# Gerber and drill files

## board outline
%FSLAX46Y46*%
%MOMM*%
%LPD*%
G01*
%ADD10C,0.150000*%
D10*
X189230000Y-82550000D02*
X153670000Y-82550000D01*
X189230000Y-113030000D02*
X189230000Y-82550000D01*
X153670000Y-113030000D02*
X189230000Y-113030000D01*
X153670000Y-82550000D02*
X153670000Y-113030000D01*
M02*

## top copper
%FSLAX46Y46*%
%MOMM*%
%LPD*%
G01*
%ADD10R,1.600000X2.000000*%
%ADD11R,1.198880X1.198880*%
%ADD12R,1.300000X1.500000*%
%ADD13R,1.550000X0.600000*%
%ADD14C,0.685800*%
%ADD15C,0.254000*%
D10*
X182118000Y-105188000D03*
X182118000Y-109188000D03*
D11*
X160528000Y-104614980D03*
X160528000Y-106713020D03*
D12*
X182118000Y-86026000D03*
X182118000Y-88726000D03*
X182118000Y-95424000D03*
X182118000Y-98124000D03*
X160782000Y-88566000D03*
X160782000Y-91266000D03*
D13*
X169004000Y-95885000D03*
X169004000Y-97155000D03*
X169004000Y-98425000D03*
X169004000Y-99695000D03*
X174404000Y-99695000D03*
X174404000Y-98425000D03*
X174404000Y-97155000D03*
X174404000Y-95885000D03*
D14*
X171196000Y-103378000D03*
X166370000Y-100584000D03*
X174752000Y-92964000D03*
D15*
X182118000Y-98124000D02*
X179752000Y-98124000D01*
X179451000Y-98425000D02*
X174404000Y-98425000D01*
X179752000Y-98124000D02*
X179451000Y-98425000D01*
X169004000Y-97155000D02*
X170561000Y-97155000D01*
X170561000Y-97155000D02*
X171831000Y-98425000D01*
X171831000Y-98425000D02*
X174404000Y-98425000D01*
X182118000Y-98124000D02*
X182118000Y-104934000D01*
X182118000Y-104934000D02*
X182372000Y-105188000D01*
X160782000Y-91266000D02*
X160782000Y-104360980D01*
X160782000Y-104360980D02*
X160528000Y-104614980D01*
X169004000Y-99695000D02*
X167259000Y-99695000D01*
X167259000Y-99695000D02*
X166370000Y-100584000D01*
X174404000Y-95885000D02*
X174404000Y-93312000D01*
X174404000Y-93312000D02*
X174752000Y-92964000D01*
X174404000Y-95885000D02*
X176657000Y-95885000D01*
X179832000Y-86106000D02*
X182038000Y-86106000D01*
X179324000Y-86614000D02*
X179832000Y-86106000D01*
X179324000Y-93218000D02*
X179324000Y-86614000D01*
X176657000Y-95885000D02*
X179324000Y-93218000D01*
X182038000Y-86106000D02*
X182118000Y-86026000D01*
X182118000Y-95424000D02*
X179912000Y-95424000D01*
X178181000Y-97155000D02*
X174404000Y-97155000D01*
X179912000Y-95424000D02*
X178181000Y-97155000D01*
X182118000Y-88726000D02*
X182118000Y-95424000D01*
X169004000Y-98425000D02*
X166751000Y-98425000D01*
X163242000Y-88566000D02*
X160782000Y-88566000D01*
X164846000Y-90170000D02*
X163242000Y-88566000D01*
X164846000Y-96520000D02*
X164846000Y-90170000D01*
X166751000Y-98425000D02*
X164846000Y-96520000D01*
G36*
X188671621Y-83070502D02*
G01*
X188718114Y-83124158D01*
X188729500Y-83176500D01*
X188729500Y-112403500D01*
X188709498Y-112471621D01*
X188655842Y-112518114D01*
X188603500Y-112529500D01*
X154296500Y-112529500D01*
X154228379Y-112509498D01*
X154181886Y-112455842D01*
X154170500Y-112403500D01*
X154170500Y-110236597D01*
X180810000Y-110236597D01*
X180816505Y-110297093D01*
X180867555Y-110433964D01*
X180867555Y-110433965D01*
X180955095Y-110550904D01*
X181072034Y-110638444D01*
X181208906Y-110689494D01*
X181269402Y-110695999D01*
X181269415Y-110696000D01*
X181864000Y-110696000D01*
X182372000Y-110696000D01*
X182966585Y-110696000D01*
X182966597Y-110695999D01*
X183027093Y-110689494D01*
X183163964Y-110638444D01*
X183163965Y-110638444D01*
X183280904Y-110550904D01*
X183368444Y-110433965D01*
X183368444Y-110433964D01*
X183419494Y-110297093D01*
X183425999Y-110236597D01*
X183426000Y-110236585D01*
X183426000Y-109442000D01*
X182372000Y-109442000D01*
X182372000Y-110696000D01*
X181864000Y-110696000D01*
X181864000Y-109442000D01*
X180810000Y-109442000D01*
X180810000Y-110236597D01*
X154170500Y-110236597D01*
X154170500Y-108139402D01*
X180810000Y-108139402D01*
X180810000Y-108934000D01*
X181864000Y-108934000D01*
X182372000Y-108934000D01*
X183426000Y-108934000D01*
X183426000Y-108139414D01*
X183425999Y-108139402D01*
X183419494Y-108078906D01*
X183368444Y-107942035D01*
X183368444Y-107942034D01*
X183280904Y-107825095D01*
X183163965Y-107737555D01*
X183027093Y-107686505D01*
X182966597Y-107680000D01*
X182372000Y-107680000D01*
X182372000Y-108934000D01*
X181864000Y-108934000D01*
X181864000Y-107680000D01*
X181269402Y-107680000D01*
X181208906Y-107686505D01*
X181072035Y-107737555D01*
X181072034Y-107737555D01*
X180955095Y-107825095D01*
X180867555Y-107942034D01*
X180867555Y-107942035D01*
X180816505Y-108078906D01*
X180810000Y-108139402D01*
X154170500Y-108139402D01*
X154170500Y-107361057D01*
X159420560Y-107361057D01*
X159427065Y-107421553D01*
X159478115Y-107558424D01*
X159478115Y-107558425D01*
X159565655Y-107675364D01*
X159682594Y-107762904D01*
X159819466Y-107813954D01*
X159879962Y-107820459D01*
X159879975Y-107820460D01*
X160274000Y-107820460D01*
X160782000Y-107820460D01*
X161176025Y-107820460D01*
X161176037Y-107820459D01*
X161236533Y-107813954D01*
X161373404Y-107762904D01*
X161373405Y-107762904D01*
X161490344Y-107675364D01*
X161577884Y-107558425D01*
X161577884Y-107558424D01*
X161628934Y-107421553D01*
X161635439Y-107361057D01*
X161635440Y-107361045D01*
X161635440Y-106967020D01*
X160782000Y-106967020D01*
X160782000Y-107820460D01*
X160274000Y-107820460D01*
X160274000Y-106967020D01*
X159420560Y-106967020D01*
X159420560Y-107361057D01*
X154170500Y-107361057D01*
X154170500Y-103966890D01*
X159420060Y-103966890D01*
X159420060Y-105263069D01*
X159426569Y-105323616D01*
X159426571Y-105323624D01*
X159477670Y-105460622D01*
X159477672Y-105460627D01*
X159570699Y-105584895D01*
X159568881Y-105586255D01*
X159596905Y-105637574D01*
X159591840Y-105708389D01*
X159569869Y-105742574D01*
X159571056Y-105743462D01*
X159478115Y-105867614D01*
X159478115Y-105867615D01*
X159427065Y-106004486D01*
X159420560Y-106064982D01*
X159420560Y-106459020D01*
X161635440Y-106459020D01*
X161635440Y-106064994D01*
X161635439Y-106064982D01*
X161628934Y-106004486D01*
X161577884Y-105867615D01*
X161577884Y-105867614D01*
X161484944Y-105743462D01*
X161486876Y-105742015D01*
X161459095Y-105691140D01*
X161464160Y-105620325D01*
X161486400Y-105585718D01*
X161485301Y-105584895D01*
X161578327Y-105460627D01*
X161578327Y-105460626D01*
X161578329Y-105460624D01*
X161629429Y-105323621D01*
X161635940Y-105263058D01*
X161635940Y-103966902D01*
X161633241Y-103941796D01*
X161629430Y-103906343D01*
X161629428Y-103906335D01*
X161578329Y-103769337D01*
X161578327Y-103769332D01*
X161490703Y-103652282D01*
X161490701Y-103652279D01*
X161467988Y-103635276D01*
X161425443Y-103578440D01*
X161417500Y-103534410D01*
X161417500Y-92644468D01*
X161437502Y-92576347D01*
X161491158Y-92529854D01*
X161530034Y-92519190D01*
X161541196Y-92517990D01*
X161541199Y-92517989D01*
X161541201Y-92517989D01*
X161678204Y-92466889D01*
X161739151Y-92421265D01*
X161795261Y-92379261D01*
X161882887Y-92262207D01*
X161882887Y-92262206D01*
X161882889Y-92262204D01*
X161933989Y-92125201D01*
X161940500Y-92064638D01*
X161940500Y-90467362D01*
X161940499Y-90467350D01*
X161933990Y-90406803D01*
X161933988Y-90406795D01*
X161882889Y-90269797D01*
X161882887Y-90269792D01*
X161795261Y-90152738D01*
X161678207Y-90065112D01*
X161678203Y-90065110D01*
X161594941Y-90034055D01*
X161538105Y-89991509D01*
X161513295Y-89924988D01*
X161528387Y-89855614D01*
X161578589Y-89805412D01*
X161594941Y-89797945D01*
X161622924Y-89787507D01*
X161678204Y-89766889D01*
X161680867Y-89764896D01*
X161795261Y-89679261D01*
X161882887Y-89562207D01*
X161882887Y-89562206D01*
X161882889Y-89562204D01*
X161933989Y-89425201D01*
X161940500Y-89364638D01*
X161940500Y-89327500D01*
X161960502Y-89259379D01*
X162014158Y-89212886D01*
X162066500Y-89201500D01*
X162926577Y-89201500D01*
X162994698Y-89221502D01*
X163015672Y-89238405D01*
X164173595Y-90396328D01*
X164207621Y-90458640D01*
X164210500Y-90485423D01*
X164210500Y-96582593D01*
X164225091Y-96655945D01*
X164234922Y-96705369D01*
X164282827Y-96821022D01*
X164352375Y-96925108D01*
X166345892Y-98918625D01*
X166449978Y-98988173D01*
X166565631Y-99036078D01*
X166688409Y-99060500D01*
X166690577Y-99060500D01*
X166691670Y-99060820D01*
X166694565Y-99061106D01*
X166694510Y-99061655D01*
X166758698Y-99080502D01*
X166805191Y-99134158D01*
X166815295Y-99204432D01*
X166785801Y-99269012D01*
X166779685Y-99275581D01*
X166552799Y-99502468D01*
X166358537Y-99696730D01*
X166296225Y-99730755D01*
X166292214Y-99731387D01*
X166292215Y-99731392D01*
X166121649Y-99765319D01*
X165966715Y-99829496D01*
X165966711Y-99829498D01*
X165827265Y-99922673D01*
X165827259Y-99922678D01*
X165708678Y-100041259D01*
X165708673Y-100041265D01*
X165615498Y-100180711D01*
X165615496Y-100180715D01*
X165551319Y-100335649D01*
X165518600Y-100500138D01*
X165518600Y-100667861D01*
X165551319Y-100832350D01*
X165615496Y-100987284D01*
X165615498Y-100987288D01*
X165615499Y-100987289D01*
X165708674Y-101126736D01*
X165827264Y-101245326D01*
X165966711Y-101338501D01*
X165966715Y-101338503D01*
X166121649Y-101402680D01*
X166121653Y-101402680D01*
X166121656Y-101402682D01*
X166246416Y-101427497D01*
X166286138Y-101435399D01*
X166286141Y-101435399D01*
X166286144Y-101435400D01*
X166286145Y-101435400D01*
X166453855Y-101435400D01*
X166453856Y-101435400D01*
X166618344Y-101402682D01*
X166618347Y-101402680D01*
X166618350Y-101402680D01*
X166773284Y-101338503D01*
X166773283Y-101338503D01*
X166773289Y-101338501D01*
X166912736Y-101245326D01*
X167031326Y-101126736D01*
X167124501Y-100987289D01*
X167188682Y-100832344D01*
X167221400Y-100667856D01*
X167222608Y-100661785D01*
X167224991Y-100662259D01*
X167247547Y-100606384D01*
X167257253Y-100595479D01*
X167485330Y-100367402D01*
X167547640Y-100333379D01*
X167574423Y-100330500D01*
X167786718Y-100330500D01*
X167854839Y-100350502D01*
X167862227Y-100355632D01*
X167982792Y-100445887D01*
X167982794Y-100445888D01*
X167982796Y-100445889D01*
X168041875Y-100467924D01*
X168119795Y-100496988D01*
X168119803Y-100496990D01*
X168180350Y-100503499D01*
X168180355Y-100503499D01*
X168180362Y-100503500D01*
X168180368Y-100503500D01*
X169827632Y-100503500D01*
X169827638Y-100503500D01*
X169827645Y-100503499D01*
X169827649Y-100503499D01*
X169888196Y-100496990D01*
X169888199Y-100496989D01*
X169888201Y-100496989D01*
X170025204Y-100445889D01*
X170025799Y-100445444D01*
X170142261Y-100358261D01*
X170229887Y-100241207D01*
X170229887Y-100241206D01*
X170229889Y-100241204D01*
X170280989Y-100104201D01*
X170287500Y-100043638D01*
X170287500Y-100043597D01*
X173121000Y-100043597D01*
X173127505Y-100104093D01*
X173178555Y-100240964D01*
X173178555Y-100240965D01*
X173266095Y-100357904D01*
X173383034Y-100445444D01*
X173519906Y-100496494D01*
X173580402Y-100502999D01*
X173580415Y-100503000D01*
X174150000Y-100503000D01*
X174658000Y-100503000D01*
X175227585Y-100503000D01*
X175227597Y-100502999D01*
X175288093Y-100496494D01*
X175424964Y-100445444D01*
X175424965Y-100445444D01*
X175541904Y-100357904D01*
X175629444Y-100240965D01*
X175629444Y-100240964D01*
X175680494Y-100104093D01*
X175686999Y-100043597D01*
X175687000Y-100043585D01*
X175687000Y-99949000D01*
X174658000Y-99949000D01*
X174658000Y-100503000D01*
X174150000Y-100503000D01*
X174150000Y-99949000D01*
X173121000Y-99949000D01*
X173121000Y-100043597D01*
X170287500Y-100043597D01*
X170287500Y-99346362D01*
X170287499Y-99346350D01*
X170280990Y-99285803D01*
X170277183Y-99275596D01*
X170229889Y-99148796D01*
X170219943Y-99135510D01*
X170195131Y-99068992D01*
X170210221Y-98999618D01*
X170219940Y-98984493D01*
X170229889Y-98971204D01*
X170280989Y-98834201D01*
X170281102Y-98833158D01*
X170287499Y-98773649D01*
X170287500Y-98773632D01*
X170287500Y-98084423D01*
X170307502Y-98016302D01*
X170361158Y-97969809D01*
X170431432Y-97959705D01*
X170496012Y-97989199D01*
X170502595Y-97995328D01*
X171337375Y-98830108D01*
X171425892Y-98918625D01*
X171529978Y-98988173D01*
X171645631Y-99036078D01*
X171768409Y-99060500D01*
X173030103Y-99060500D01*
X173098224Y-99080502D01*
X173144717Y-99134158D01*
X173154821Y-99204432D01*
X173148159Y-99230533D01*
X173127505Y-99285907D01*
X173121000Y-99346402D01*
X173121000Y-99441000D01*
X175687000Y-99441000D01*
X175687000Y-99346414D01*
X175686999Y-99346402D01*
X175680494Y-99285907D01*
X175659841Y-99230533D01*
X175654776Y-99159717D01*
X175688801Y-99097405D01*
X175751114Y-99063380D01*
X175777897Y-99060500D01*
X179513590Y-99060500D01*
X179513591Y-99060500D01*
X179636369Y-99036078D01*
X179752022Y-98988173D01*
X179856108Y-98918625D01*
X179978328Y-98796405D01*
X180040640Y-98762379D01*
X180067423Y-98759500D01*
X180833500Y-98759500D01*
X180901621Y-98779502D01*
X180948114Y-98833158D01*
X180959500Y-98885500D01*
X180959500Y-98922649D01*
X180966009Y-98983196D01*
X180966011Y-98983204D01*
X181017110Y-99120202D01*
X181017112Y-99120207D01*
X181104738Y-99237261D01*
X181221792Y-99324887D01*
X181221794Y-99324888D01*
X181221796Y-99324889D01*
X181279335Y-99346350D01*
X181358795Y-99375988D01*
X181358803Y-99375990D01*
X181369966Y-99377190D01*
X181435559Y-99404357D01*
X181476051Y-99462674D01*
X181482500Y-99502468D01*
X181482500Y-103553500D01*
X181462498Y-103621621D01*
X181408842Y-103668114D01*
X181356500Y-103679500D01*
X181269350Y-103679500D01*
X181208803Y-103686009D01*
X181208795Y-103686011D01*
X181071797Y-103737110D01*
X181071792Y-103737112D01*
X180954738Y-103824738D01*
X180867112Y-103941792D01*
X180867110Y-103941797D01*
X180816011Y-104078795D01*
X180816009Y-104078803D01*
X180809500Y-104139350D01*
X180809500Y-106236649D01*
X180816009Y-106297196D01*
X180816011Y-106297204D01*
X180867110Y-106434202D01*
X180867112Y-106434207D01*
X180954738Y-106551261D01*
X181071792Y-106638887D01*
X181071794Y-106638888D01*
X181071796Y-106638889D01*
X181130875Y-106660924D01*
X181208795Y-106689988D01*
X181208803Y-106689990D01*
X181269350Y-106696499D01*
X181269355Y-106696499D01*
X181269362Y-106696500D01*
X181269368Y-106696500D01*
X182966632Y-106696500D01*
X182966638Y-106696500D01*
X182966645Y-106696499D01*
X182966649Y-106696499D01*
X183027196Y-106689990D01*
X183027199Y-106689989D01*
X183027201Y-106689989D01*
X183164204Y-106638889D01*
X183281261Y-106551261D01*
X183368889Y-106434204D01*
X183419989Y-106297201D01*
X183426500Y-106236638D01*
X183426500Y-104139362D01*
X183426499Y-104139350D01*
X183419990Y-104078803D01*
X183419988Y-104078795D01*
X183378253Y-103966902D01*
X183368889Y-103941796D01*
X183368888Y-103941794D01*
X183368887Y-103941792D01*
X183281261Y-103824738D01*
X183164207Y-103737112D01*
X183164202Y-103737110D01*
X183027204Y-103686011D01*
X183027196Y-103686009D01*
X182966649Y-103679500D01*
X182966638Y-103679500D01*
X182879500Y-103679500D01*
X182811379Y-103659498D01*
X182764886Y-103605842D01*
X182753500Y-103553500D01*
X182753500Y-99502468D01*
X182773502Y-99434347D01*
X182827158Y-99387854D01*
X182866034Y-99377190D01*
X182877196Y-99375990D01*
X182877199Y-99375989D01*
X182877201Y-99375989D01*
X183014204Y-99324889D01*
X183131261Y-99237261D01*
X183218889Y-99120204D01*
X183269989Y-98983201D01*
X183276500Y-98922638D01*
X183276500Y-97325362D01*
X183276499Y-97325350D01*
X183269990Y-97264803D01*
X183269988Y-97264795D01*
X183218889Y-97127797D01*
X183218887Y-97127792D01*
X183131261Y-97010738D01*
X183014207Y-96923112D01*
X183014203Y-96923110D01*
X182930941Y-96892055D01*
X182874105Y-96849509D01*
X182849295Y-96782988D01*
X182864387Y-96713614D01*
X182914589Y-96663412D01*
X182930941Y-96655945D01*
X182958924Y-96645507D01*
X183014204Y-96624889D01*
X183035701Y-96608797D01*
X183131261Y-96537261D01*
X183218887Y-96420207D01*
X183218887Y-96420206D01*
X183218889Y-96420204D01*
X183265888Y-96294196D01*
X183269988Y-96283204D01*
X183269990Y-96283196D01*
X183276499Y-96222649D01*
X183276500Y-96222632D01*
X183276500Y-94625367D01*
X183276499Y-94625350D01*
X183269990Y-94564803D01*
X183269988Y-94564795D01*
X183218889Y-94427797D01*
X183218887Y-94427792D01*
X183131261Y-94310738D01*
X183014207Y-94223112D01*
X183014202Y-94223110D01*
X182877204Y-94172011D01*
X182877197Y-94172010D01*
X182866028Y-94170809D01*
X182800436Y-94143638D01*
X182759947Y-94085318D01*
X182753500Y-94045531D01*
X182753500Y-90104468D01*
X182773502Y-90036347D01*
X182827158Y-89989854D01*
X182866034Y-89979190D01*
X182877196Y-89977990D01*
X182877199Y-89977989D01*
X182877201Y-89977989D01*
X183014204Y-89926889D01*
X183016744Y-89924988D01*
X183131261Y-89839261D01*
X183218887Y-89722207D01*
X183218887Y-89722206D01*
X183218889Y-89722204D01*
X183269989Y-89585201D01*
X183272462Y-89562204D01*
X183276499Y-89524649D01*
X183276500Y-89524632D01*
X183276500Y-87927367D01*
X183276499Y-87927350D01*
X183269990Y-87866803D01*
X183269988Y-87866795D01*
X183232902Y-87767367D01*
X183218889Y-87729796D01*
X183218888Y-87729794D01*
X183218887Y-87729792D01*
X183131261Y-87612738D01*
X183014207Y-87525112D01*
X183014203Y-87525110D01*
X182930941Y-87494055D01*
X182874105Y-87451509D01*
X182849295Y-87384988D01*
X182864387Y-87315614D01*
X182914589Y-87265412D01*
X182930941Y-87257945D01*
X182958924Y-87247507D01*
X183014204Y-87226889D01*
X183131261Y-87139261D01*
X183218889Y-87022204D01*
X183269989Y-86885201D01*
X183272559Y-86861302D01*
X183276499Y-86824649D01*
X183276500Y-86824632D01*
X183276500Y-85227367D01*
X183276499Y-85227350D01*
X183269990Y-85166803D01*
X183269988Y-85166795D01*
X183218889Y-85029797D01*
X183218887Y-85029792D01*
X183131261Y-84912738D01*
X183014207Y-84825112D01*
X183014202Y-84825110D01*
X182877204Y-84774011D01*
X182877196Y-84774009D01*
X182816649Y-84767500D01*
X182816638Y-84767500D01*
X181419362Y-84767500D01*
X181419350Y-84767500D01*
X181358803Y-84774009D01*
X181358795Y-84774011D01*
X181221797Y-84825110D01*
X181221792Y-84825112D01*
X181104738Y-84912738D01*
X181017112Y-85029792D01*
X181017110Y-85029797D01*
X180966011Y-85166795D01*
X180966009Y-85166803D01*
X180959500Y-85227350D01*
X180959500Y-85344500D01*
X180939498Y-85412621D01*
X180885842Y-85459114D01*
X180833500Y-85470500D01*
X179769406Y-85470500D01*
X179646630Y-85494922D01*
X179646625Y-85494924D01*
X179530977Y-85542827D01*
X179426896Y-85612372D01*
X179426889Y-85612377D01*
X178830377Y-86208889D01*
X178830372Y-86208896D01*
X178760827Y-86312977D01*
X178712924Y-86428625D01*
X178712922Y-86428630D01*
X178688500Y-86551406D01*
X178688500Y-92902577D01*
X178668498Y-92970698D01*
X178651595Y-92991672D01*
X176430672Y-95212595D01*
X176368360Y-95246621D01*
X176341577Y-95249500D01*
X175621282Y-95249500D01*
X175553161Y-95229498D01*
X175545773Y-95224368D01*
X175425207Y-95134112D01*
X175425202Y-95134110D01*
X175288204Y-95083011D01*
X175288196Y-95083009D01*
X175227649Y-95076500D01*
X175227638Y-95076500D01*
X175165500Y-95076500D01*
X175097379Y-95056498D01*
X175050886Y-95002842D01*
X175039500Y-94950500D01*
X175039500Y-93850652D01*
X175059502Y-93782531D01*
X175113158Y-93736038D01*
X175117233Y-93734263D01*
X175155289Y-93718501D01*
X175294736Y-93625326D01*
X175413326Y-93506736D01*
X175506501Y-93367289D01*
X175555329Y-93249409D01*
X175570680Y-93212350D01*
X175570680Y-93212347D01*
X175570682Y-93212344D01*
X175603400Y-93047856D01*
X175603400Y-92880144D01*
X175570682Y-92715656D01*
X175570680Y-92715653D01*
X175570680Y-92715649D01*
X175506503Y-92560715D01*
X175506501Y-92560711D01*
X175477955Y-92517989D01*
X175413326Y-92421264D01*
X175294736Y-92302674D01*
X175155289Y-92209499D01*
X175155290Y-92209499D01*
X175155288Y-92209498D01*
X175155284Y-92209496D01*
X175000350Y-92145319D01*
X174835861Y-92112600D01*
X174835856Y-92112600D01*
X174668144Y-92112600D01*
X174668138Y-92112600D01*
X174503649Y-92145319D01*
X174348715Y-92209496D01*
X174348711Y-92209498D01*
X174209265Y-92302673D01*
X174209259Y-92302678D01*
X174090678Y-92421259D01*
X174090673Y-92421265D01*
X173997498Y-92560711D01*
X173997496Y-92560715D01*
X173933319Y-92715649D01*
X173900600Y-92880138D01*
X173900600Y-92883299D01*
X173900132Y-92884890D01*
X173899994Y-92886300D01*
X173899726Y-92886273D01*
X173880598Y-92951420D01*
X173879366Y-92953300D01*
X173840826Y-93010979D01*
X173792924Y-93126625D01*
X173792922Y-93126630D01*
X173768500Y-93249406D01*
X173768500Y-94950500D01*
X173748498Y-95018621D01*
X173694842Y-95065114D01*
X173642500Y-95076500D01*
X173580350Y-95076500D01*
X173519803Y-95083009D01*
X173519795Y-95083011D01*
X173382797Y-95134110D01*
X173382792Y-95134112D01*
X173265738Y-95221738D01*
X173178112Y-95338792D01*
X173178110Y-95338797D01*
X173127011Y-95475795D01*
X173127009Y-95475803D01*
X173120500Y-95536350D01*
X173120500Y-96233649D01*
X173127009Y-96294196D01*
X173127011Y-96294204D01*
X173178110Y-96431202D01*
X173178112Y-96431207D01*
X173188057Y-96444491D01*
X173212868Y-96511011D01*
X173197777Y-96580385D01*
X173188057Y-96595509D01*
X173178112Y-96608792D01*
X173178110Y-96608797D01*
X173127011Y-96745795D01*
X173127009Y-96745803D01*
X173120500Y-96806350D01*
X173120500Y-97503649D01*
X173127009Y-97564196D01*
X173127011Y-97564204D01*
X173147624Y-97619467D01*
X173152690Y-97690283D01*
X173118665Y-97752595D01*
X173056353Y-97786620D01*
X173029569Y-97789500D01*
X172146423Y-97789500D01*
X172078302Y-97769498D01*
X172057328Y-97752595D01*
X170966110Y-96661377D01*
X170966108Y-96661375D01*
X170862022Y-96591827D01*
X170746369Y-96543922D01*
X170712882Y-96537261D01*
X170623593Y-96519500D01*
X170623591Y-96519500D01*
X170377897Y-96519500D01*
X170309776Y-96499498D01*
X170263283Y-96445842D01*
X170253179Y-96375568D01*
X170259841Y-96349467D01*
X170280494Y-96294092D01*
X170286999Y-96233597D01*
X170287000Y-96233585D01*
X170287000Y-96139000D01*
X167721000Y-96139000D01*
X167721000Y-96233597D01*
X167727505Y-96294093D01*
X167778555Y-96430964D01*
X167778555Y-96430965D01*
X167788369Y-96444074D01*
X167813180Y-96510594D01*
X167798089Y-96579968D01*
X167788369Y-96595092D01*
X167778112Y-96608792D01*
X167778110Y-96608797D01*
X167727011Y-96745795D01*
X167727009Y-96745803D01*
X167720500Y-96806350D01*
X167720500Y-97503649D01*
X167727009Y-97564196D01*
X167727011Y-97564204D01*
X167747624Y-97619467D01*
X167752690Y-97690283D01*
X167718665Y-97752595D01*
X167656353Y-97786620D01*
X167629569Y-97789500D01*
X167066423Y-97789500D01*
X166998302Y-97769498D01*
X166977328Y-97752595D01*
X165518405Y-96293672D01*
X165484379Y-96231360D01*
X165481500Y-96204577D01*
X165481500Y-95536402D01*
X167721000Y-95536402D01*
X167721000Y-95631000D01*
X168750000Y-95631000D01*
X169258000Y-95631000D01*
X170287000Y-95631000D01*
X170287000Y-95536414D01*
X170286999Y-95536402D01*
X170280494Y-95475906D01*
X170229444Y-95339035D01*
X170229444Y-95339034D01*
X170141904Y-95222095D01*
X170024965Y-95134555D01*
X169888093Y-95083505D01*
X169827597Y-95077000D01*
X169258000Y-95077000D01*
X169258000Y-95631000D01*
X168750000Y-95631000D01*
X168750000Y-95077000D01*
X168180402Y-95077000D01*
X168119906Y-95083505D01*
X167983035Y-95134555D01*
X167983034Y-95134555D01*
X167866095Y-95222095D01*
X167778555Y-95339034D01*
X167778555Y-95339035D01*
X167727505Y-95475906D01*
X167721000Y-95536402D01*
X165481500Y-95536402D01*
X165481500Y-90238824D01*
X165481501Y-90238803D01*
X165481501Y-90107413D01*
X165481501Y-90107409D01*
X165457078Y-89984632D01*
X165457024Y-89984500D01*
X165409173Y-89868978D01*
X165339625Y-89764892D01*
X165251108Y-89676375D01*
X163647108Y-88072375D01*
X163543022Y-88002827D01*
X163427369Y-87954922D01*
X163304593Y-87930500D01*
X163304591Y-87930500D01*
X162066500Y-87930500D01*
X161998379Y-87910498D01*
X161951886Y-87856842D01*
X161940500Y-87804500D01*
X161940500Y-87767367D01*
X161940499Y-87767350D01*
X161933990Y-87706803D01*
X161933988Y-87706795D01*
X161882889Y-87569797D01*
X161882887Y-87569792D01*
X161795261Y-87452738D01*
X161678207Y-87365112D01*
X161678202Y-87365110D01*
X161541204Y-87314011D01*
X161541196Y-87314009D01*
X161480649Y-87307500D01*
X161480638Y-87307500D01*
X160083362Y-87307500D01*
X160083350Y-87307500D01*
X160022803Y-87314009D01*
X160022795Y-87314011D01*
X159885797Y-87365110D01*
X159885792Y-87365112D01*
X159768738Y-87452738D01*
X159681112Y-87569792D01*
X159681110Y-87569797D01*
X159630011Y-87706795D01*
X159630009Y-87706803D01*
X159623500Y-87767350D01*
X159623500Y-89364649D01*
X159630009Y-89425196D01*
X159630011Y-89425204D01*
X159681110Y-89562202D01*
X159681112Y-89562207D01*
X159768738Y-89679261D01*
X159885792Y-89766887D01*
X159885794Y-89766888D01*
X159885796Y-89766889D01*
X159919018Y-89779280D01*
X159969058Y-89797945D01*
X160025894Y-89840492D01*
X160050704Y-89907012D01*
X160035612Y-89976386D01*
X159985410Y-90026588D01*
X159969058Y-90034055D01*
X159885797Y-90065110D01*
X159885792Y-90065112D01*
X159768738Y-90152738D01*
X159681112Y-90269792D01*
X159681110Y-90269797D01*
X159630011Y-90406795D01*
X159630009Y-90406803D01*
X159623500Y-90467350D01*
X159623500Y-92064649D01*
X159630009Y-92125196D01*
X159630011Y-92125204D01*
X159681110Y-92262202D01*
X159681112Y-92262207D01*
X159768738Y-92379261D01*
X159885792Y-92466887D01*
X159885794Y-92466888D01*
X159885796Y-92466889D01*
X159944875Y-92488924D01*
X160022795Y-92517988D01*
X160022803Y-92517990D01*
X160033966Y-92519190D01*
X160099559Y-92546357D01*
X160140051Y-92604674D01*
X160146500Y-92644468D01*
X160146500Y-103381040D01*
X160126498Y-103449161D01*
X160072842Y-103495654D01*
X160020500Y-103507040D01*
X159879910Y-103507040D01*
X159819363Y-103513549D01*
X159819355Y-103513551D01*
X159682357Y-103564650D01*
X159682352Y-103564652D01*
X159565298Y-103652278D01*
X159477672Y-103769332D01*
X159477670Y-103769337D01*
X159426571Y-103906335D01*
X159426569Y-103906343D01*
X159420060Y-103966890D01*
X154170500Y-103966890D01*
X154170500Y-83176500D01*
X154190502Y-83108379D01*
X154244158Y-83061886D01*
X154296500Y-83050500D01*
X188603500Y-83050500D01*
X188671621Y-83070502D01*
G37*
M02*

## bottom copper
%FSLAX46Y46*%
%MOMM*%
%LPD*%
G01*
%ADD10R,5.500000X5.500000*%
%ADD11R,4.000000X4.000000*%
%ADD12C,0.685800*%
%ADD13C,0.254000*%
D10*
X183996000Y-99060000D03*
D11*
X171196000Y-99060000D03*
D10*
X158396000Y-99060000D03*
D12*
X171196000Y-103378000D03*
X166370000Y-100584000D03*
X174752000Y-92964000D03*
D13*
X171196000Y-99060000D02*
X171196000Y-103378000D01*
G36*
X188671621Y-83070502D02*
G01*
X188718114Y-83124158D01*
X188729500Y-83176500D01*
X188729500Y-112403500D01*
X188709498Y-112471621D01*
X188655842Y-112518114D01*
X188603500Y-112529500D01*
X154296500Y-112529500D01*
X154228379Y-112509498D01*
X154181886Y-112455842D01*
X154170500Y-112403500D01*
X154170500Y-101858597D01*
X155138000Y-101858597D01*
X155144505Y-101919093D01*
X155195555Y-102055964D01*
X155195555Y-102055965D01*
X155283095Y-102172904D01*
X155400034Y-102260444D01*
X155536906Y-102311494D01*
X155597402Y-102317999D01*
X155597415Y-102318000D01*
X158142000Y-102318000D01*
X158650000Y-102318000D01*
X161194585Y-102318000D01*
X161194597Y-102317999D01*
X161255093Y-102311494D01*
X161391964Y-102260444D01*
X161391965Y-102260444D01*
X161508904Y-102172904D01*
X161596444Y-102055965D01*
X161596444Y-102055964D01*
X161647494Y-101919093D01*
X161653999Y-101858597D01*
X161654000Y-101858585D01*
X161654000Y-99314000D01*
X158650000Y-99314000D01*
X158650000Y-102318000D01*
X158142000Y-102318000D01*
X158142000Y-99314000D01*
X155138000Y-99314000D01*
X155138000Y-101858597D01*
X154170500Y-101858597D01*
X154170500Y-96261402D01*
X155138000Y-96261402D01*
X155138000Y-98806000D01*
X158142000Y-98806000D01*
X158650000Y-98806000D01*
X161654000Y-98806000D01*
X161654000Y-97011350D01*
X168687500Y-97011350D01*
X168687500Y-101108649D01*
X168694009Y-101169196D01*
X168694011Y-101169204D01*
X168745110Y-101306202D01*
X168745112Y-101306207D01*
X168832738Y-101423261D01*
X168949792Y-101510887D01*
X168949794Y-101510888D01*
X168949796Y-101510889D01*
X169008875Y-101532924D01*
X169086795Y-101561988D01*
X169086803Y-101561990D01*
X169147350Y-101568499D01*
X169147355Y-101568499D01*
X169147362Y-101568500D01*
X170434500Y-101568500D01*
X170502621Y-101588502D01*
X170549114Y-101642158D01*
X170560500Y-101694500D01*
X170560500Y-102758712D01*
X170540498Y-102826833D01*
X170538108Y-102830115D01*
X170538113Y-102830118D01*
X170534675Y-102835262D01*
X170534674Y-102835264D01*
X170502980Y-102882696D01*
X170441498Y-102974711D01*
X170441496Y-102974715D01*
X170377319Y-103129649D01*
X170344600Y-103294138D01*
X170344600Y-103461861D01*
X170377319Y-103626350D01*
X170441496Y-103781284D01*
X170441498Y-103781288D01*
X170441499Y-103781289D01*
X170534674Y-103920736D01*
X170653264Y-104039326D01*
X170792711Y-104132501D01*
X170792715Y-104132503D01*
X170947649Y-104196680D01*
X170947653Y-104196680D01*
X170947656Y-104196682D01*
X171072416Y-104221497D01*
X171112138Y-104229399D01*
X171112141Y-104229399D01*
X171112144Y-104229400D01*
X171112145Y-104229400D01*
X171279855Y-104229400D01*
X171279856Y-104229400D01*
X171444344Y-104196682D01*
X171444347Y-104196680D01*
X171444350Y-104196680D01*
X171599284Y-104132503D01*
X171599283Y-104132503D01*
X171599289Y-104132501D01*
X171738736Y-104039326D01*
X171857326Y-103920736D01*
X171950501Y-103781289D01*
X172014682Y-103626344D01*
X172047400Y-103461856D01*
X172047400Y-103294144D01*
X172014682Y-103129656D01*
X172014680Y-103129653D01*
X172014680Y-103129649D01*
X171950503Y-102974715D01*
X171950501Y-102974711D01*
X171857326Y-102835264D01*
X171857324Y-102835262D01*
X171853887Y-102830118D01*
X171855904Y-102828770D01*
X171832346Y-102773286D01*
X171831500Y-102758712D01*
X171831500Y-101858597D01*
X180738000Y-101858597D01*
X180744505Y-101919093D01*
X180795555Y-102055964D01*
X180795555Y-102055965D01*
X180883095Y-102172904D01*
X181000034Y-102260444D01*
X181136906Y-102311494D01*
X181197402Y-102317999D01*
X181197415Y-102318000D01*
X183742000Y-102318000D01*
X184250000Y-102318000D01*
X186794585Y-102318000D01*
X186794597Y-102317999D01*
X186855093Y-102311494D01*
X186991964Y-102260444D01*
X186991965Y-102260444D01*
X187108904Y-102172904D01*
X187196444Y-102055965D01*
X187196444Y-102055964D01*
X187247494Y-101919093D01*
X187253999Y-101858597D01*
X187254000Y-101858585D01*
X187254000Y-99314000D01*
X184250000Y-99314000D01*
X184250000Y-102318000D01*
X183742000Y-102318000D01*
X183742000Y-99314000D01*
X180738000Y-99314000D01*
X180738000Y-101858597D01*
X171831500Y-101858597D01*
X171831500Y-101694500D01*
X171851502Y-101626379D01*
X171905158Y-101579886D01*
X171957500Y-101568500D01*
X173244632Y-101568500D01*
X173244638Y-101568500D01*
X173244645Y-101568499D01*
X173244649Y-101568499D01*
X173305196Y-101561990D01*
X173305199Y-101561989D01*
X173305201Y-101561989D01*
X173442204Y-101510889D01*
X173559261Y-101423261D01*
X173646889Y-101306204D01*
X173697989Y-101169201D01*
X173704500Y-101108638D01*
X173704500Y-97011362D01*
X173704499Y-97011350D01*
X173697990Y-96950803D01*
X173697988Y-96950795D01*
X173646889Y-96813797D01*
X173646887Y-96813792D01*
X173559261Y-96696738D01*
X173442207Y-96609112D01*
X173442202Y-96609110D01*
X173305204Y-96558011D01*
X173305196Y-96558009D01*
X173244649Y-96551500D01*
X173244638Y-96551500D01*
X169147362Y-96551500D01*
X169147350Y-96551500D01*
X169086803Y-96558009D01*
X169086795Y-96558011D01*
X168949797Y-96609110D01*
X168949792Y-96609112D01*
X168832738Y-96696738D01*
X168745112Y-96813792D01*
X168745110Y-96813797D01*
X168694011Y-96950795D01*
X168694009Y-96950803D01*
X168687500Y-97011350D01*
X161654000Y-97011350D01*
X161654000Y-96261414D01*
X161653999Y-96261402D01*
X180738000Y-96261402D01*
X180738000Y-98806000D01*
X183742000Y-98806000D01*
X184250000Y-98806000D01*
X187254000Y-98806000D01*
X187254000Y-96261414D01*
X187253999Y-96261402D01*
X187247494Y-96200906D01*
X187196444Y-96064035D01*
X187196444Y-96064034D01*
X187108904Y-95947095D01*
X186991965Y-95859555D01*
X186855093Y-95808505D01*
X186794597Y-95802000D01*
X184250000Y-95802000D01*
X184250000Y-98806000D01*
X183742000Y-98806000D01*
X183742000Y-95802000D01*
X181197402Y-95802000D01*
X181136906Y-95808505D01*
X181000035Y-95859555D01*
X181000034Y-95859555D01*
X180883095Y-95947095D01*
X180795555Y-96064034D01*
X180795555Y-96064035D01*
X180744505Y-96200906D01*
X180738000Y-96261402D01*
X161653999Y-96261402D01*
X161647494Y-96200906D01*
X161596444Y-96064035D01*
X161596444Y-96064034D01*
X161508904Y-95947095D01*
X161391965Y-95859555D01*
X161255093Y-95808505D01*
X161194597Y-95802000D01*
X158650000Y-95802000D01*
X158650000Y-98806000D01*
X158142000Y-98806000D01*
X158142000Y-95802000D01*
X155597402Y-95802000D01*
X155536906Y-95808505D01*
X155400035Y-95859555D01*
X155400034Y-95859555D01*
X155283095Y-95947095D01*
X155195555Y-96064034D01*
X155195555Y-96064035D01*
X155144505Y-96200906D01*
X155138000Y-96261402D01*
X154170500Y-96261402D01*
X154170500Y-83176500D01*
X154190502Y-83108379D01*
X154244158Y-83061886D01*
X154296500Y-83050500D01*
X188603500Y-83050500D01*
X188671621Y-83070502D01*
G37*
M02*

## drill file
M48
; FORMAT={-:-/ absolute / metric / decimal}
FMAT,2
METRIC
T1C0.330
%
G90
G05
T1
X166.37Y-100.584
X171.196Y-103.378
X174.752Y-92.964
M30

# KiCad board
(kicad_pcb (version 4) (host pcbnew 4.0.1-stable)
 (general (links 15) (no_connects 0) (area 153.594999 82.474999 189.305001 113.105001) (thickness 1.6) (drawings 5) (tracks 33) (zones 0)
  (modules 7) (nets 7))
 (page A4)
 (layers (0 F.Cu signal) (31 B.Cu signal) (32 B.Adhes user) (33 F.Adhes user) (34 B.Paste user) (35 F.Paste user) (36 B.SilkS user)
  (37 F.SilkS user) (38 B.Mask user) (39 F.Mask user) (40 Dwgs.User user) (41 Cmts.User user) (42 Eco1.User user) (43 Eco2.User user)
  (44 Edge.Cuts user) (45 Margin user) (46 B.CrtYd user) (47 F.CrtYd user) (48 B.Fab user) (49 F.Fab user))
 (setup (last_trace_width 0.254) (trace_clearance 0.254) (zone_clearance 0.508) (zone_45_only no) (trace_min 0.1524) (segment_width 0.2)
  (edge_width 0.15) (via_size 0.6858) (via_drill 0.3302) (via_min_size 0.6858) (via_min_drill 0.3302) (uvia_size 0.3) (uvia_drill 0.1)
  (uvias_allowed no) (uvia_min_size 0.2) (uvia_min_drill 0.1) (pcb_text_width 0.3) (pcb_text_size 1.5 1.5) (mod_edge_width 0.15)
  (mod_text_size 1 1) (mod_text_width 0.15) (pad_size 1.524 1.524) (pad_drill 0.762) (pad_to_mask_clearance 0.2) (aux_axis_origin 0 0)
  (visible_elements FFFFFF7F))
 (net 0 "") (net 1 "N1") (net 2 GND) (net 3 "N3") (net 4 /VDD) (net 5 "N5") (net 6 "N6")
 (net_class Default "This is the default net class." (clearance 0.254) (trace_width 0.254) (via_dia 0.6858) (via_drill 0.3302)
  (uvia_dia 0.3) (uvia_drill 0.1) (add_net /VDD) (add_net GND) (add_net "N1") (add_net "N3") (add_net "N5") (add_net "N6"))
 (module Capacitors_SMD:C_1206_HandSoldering (layer F.Cu) (at 182.118 107.188 270)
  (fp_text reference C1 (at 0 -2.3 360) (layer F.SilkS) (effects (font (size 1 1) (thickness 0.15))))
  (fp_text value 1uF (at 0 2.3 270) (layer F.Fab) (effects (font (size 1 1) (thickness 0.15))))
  (pad 1 smd rect (at -2 0 270) (size 2 1.6) (layers F.Cu F.Paste F.Mask) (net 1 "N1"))
  (pad 2 smd rect (at 2 0 270) (size 2 1.6) (layers F.Cu F.Paste F.Mask) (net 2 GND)))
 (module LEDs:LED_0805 (layer F.Cu) (at 160.528 105.664 90)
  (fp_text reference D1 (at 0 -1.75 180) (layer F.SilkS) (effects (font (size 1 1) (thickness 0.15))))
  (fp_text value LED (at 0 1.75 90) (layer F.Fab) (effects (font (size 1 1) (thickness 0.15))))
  (pad 2 smd rect (at 1.04902 0 270) (size 1.19888 1.19888) (layers F.Cu F.Paste F.Mask) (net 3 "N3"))
  (pad 1 smd rect (at -1.04902 0 270) (size 1.19888 1.19888) (layers F.Cu F.Paste F.Mask) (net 2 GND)))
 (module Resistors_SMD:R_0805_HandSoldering (layer F.Cu) (at 182.118 87.376 270)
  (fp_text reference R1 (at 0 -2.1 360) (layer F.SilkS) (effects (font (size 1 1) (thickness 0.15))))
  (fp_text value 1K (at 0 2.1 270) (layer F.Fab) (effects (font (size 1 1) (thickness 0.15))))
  (pad 1 smd rect (at -1.35 0 270) (size 1.5 1.3) (layers F.Cu F.Paste F.Mask) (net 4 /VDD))
  (pad 2 smd rect (at 1.35 0 270) (size 1.5 1.3) (layers F.Cu F.Paste F.Mask) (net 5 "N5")))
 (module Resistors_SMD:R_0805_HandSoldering (layer F.Cu) (at 182.118 96.774 270)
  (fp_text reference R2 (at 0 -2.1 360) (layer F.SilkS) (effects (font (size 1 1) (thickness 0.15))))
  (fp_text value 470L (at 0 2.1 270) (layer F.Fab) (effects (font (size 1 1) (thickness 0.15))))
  (pad 1 smd rect (at -1.35 0 270) (size 1.5 1.3) (layers F.Cu F.Paste F.Mask) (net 5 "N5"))
  (pad 2 smd rect (at 1.35 0 270) (size 1.5 1.3) (layers F.Cu F.Paste F.Mask) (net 1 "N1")))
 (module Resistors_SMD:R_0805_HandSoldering (layer F.Cu) (at 160.782 89.916 270)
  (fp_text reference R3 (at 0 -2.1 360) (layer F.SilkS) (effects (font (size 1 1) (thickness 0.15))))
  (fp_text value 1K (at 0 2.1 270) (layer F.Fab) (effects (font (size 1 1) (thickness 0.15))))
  (pad 1 smd rect (at -1.35 0 270) (size 1.5 1.3) (layers F.Cu F.Paste F.Mask) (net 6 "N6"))
  (pad 2 smd rect (at 1.35 0 270) (size 1.5 1.3) (layers F.Cu F.Paste F.Mask) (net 3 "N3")))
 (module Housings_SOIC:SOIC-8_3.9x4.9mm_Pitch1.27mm (layer F.Cu) (at 171.704 97.79)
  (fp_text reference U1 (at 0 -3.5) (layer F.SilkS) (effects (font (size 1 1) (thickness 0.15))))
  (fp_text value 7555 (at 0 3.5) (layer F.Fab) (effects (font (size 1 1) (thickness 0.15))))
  (pad 1 smd rect (at -2.7 -1.905) (size 1.55 0.6) (layers F.Cu F.Paste F.Mask) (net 2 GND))
  (pad 2 smd rect (at -2.7 -0.635) (size 1.55 0.6) (layers F.Cu F.Paste F.Mask) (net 1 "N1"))
  (pad 3 smd rect (at -2.7 0.635) (size 1.55 0.6) (layers F.Cu F.Paste F.Mask) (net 6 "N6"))
  (pad 4 smd rect (at -2.7 1.905) (size 1.55 0.6) (layers F.Cu F.Paste F.Mask) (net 4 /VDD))
  (pad 5 smd rect (at 2.7 1.905) (size 1.55 0.6) (layers F.Cu F.Paste F.Mask) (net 2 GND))
  (pad 6 smd rect (at 2.7 0.635) (size 1.55 0.6) (layers F.Cu F.Paste F.Mask) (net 1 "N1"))
  (pad 7 smd rect (at 2.7 -0.635) (size 1.55 0.6) (layers F.Cu F.Paste F.Mask) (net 5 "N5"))
  (pad 8 smd rect (at 2.7 -1.905) (size 1.55 0.6) (layers F.Cu F.Paste F.Mask) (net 4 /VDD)))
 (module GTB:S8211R (layer B.Cu) (at 171.196 99.06)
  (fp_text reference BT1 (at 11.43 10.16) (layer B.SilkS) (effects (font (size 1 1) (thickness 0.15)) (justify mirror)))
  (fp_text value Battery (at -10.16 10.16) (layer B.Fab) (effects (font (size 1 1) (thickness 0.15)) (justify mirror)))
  (pad 1 smd rect (at 12.8 0) (size 5.5 5.5) (layers B.Cu B.Paste B.Mask) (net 4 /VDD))
  (pad 2 smd rect (at 0 0) (size 4 4) (layers B.Cu B.Paste B.Mask) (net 2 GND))
  (pad 1 smd rect (at -12.8 0) (size 5.5 5.5) (layers B.Cu B.Paste B.Mask) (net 4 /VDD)))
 (gr_line (start 189.23 82.55) (end 153.67 82.55) (angle 90) (layer Edge.Cuts) (width 0.15))
 (gr_line (start 189.23 113.03) (end 189.23 82.55) (angle 90) (layer Edge.Cuts) (width 0.15))
 (gr_line (start 153.67 113.03) (end 189.23 113.03) (angle 90) (layer Edge.Cuts) (width 0.15))
 (gr_line (start 153.67 82.55) (end 153.67 113.03) (angle 90) (layer Edge.Cuts) (width 0.15))
 (segment (start 182.118 98.124) (end 179.752 98.124) (width 0.254) (layer F.Cu) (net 1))
 (segment (start 179.451 98.425) (end 174.404 98.425) (width 0.254) (layer F.Cu) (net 1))
 (segment (start 179.752 98.124) (end 179.451 98.425) (width 0.254) (layer F.Cu) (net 1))
 (segment (start 169.004 97.155) (end 170.561 97.155) (width 0.254) (layer F.Cu) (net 1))
 (segment (start 170.561 97.155) (end 171.831 98.425) (width 0.254) (layer F.Cu) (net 1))
 (segment (start 171.831 98.425) (end 174.404 98.425) (width 0.254) (layer F.Cu) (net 1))
 (segment (start 182.118 98.124) (end 182.118 104.934) (width 0.254) (layer F.Cu) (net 1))
 (segment (start 182.118 104.934) (end 182.372 105.188) (width 0.254) (layer F.Cu) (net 1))
 (segment (start 171.196 99.06) (end 171.196 103.378) (width 0.254) (layer B.Cu) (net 2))
 (via (at 171.196 103.378) (size 0.6858) (drill 0.3302) (layers F.Cu B.Cu) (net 2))
 (segment (start 160.782 91.266) (end 160.782 104.36098) (width 0.254) (layer F.Cu) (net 3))
 (segment (start 160.782 104.36098) (end 160.528 104.61498) (width 0.254) (layer F.Cu) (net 3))
 (segment (start 169.004 99.695) (end 167.259 99.695) (width 0.254) (layer F.Cu) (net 4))
 (via (at 166.37 100.584) (size 0.6858) (drill 0.3302) (layers F.Cu B.Cu) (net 4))
 (segment (start 167.259 99.695) (end 166.37 100.584) (width 0.254) (layer F.Cu) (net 4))
 (segment (start 174.404 95.885) (end 174.404 93.312) (width 0.254) (layer F.Cu) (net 4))
 (via (at 174.752 92.964) (size 0.6858) (drill 0.3302) (layers F.Cu B.Cu) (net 4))
 (segment (start 174.404 93.312) (end 174.752 92.964) (width 0.254) (layer F.Cu) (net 4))
 (segment (start 174.404 95.885) (end 176.657 95.885) (width 0.254) (layer F.Cu) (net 4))
 (segment (start 179.832 86.106) (end 182.038 86.106) (width 0.254) (layer F.Cu) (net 4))
 (segment (start 179.324 86.614) (end 179.832 86.106) (width 0.254) (layer F.Cu) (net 4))
 (segment (start 179.324 93.218) (end 179.324 86.614) (width 0.254) (layer F.Cu) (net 4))
 (segment (start 176.657 95.885) (end 179.324 93.218) (width 0.254) (layer F.Cu) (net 4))
 (segment (start 182.038 86.106) (end 182.118 86.026) (width 0.254) (layer F.Cu) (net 4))
 (segment (start 182.118 95.424) (end 179.912 95.424) (width 0.254) (layer F.Cu) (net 5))
 (segment (start 178.181 97.155) (end 174.404 97.155) (width 0.254) (layer F.Cu) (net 5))
 (segment (start 179.912 95.424) (end 178.181 97.155) (width 0.254) (layer F.Cu) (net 5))
 (segment (start 182.118 88.726) (end 182.118 95.424) (width 0.254) (layer F.Cu) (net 5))
 (segment (start 169.004 98.425) (end 166.751 98.425) (width 0.254) (layer F.Cu) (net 6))
 (segment (start 163.242 88.566) (end 160.782 88.566) (width 0.254) (layer F.Cu) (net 6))
 (segment (start 164.846 90.17) (end 163.242 88.566) (width 0.254) (layer F.Cu) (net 6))
 (segment (start 164.846 96.52) (end 164.846 90.17) (width 0.254) (layer F.Cu) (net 6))
 (segment (start 166.751 98.425) (end 164.846 96.52) (width 0.254) (layer F.Cu) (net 6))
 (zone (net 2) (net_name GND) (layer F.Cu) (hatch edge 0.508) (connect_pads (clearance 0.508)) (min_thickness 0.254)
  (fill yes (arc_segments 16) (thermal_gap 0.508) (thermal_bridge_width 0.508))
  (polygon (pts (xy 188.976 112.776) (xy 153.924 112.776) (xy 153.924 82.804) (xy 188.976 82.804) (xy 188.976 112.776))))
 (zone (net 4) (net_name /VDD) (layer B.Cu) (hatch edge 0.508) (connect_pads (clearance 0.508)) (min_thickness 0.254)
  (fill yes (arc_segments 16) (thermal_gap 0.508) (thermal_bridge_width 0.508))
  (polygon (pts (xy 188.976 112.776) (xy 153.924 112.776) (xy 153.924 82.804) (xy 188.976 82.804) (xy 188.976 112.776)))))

